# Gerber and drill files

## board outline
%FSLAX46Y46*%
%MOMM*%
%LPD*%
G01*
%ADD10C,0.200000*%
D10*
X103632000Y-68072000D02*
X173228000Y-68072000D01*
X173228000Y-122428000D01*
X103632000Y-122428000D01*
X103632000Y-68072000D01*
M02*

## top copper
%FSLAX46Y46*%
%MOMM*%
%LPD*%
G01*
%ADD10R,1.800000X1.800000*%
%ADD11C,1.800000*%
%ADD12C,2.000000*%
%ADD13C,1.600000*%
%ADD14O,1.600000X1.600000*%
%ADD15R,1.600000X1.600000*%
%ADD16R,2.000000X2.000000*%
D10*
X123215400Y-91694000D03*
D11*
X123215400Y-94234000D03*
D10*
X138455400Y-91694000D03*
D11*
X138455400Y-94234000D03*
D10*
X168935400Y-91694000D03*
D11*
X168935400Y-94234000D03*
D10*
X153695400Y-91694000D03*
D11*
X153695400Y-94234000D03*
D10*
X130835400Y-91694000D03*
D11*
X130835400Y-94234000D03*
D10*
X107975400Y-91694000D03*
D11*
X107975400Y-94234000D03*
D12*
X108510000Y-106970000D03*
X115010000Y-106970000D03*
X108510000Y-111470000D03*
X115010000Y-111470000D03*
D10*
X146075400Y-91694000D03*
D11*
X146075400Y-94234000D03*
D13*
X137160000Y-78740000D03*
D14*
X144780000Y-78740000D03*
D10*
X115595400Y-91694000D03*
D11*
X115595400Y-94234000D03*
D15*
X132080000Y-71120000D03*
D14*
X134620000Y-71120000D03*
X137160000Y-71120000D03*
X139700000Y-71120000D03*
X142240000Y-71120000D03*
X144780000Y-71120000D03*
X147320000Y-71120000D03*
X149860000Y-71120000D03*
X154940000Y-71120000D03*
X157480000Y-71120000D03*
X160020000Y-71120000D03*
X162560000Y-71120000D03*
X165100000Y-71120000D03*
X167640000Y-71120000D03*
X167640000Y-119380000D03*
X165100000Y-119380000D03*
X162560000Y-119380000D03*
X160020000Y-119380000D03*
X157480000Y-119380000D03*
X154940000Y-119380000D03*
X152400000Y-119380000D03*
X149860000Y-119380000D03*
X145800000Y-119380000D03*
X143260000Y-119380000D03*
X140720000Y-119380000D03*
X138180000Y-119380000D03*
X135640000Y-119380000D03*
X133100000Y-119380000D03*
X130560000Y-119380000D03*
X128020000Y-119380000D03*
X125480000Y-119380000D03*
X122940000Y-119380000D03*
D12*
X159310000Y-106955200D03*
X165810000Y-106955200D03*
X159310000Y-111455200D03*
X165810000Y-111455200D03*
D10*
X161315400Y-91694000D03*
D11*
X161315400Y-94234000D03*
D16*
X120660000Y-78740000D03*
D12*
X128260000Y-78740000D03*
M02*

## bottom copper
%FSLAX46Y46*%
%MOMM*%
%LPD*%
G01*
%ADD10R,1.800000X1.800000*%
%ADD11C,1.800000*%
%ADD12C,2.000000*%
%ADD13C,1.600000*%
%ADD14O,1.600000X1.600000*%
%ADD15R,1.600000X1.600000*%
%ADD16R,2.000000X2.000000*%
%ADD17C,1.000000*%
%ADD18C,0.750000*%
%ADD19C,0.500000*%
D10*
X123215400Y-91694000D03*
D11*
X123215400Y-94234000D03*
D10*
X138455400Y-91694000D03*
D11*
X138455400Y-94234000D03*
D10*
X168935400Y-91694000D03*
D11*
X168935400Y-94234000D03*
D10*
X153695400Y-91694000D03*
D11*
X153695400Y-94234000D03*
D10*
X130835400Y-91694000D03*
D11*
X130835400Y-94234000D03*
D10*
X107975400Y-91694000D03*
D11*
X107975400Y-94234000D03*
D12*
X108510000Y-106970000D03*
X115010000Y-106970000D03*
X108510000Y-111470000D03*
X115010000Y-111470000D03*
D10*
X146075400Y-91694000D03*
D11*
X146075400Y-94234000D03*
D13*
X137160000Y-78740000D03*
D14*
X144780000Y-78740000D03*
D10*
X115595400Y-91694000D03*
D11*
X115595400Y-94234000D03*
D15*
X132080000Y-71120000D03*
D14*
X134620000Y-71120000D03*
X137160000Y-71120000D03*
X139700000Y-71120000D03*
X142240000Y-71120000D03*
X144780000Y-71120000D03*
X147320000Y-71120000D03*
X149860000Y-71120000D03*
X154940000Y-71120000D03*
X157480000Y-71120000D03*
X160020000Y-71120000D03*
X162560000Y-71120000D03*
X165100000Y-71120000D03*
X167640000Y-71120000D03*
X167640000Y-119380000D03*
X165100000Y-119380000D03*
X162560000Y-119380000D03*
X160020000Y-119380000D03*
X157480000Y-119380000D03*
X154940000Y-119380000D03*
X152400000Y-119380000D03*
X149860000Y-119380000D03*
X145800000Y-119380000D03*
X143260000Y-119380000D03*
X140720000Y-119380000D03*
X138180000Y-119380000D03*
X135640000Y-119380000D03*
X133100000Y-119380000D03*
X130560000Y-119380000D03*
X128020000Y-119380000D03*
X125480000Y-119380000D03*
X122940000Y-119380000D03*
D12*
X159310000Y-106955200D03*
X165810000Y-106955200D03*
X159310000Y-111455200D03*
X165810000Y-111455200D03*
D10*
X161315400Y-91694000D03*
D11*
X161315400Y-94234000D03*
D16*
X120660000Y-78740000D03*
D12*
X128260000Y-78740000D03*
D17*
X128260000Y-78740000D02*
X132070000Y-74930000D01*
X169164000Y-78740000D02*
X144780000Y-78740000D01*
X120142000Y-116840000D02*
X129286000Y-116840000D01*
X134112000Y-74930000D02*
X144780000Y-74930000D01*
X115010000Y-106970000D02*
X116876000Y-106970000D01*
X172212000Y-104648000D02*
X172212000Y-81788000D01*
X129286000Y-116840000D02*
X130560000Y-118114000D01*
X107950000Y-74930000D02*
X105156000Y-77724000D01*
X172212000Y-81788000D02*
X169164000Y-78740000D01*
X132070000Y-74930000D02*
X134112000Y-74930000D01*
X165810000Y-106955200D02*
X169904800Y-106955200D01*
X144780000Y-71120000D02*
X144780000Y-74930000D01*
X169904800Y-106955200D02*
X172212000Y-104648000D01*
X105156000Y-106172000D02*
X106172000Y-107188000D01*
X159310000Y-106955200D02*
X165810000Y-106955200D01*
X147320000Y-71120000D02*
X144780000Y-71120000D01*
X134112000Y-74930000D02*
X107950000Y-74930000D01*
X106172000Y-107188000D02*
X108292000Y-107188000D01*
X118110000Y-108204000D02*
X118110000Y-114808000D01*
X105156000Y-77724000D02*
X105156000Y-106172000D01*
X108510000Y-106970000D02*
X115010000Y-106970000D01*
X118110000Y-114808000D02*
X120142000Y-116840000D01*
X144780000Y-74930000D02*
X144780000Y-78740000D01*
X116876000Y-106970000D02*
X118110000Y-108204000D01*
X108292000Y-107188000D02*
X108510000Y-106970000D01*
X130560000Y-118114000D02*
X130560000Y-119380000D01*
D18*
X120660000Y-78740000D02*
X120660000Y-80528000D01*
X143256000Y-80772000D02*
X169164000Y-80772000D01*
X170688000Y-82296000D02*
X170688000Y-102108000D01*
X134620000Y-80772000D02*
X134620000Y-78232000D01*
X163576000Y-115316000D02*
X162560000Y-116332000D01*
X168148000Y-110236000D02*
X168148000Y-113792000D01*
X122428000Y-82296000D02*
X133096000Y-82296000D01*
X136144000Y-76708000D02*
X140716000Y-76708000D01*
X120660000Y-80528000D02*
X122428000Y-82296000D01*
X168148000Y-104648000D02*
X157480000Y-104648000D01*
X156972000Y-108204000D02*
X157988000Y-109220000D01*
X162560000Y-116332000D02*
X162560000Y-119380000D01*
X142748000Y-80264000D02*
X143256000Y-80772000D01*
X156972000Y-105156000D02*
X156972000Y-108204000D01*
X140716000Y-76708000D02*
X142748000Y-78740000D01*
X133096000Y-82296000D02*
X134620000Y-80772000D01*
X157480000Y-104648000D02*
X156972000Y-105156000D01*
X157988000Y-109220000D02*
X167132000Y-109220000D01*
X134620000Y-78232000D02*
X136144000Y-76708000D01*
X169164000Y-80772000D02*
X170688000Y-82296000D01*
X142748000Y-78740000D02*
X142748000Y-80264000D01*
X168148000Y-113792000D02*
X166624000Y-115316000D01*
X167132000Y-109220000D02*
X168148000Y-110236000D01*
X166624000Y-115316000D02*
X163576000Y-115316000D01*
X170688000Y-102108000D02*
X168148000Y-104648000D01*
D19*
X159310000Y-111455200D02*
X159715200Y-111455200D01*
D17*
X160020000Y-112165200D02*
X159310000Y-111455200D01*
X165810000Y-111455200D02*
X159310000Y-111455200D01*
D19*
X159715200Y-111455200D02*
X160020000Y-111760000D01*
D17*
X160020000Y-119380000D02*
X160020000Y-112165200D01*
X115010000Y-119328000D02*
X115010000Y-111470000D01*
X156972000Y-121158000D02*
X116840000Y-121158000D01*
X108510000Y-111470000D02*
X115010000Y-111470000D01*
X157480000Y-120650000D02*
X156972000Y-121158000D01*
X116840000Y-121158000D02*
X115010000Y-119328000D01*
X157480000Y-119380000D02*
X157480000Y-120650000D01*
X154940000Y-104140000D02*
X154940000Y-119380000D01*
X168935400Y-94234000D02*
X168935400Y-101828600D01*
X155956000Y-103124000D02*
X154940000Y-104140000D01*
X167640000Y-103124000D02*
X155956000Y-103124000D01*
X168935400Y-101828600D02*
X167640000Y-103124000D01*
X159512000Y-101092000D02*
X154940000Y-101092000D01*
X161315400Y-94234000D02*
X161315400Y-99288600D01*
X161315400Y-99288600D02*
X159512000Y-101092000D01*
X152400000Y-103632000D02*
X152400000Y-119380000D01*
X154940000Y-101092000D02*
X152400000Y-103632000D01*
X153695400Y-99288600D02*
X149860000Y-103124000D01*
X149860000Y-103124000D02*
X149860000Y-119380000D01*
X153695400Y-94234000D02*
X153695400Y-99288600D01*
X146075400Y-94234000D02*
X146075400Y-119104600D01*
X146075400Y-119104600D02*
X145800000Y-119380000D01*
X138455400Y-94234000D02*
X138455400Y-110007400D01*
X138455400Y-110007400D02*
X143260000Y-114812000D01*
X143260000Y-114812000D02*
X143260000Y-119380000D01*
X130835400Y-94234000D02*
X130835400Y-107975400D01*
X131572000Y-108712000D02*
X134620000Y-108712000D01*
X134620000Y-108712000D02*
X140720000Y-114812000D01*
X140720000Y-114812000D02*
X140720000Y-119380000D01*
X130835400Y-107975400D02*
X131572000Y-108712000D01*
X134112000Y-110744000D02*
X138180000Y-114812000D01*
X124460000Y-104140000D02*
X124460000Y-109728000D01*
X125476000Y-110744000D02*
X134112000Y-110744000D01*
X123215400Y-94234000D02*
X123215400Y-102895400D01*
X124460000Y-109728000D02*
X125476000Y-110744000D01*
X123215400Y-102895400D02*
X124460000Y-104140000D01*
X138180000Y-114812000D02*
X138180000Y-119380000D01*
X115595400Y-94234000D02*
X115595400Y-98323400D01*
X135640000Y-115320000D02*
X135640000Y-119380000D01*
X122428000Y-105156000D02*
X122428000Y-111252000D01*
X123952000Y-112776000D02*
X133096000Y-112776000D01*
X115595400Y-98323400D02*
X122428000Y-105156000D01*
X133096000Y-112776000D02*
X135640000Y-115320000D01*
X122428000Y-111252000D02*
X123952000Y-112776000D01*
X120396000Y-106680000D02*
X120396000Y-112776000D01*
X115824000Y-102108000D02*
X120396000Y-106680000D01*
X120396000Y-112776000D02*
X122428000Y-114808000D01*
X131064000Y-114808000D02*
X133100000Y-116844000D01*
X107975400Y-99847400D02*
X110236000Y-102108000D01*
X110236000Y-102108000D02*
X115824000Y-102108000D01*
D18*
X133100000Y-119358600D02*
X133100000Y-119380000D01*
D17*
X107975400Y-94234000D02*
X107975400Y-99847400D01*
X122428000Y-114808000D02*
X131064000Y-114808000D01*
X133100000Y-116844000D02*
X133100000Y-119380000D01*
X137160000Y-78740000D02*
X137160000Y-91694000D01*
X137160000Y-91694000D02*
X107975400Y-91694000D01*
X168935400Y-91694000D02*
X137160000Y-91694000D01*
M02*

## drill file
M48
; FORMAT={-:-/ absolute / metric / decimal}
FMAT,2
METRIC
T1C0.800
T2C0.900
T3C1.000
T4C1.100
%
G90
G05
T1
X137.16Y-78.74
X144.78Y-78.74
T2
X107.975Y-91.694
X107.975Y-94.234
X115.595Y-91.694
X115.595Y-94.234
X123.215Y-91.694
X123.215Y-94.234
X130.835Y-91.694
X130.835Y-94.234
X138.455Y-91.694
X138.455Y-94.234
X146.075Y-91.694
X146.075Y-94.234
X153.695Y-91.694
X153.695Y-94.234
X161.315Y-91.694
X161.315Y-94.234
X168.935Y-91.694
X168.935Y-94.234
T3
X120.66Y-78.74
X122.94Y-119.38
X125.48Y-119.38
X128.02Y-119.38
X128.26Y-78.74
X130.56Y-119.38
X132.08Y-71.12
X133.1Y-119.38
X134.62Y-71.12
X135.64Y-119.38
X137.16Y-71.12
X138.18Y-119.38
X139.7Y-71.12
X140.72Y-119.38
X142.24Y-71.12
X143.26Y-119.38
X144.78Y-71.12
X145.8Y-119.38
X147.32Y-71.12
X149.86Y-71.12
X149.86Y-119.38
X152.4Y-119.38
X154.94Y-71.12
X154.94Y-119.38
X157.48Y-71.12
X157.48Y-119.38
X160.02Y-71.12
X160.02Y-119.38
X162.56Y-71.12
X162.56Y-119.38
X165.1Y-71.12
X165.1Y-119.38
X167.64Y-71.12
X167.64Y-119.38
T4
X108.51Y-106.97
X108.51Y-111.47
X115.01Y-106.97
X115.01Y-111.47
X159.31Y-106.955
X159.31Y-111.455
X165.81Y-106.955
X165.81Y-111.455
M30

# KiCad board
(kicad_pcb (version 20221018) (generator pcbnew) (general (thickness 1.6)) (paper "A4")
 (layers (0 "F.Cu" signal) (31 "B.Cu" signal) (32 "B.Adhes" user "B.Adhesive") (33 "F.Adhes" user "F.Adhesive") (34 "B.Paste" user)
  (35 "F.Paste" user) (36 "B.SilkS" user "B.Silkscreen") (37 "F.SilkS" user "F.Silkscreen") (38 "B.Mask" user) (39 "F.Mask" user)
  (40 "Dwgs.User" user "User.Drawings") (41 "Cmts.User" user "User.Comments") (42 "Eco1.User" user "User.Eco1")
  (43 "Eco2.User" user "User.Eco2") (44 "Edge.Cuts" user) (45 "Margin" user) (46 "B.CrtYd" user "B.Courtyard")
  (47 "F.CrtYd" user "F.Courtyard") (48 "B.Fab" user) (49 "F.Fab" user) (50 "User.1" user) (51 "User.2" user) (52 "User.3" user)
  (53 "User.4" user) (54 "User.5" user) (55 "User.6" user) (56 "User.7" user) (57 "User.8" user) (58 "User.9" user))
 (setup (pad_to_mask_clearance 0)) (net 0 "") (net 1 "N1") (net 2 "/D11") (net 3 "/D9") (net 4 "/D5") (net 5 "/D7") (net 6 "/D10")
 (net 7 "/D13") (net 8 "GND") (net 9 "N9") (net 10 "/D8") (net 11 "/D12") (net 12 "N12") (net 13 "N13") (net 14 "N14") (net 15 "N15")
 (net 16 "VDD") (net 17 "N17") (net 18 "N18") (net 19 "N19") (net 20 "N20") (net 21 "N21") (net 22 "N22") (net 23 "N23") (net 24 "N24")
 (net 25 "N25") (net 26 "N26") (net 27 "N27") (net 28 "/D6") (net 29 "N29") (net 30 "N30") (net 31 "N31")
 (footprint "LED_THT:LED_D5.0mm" (layer "F.Cu") (at 123.2154 91.694 -90)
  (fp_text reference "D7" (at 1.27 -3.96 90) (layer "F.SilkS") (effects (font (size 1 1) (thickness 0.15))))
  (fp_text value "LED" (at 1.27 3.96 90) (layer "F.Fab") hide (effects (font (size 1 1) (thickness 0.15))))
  (pad "1" thru_hole rect (at 0 0 270) (size 1.8 1.8) (drill 0.9) (layers "*.Cu" "*.Mask") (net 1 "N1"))
  (pad "2" thru_hole circle (at 2.54 0 270) (size 1.8 1.8) (drill 0.9) (layers "*.Cu" "*.Mask") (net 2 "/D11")))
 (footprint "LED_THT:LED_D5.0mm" (layer "F.Cu") (at 138.4554 91.694 -90)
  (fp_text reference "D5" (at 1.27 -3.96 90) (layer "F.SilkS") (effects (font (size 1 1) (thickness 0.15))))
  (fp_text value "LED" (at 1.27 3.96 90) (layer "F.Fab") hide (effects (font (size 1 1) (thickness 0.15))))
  (pad "1" thru_hole rect (at 0 0 270) (size 1.8 1.8) (drill 0.9) (layers "*.Cu" "*.Mask") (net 1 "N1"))
  (pad "2" thru_hole circle (at 2.54 0 270) (size 1.8 1.8) (drill 0.9) (layers "*.Cu" "*.Mask") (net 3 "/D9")))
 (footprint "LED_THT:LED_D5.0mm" (layer "F.Cu") (at 168.9354 91.694 -90)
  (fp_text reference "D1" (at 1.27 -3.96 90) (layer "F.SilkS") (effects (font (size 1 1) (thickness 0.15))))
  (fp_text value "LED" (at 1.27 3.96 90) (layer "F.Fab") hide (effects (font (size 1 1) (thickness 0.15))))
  (pad "1" thru_hole rect (at 0 0 270) (size 1.8 1.8) (drill 0.9) (layers "*.Cu" "*.Mask") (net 1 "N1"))
  (pad "2" thru_hole circle (at 2.54 0 270) (size 1.8 1.8) (drill 0.9) (layers "*.Cu" "*.Mask") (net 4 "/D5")))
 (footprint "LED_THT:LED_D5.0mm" (layer "F.Cu") (at 153.6954 91.694 -90)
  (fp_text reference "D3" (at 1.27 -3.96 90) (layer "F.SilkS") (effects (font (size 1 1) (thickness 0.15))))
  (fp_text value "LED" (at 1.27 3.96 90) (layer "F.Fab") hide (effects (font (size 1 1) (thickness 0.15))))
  (pad "1" thru_hole rect (at 0 0 270) (size 1.8 1.8) (drill 0.9) (layers "*.Cu" "*.Mask") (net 1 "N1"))
  (pad "2" thru_hole circle (at 2.54 0 270) (size 1.8 1.8) (drill 0.9) (layers "*.Cu" "*.Mask") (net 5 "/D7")))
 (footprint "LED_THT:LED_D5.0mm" (layer "F.Cu") (at 130.8354 91.694 -90)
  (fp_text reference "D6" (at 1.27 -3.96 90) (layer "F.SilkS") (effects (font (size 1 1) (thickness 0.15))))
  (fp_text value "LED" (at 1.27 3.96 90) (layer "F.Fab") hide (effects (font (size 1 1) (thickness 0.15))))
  (pad "1" thru_hole rect (at 0 0 270) (size 1.8 1.8) (drill 0.9) (layers "*.Cu" "*.Mask") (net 1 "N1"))
  (pad "2" thru_hole circle (at 2.54 0 270) (size 1.8 1.8) (drill 0.9) (layers "*.Cu" "*.Mask") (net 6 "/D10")))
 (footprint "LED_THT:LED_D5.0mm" (layer "F.Cu") (at 107.9754 91.694 -90)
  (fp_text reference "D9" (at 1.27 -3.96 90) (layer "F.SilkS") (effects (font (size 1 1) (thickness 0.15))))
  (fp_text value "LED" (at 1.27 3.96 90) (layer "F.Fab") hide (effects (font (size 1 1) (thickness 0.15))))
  (pad "1" thru_hole rect (at 0 0 270) (size 1.8 1.8) (drill 0.9) (layers "*.Cu" "*.Mask") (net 1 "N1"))
  (pad "2" thru_hole circle (at 2.54 0 270) (size 1.8 1.8) (drill 0.9) (layers "*.Cu" "*.Mask") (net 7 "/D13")))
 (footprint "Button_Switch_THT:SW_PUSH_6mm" (layer "F.Cu") (at 108.51 106.97)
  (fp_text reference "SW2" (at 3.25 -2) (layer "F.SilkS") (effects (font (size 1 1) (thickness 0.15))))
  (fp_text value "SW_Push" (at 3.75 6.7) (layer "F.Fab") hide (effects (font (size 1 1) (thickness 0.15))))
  (pad "1" thru_hole circle (at 0 0 90) (size 2 2) (drill 1.1) (layers "*.Cu" "*.Mask") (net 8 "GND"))
  (pad "1" thru_hole circle (at 6.5 0 90) (size 2 2) (drill 1.1) (layers "*.Cu" "*.Mask") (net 8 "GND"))
  (pad "2" thru_hole circle (at 0 4.5 90) (size 2 2) (drill 1.1) (layers "*.Cu" "*.Mask") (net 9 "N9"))
  (pad "2" thru_hole circle (at 6.5 4.5 90) (size 2 2) (drill 1.1) (layers "*.Cu" "*.Mask") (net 9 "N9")))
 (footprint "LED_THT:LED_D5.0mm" (layer "F.Cu") (at 146.0754 91.694 -90)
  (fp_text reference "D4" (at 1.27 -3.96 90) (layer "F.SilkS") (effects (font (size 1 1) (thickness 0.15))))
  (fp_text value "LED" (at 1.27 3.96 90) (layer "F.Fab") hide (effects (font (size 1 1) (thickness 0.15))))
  (pad "1" thru_hole rect (at 0 0 270) (size 1.8 1.8) (drill 0.9) (layers "*.Cu" "*.Mask") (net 1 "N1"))
  (pad "2" thru_hole circle (at 2.54 0 270) (size 1.8 1.8) (drill 0.9) (layers "*.Cu" "*.Mask") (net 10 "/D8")))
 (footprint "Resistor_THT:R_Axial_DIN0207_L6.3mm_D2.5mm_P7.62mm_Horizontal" (layer "F.Cu") (at 137.16 78.74)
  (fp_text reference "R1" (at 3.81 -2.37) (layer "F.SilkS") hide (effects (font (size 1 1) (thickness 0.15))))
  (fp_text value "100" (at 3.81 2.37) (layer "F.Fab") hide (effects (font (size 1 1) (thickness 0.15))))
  (pad "1" thru_hole circle (at 0 0) (size 1.6 1.6) (drill 0.8) (layers "*.Cu" "*.Mask") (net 1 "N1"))
  (pad "2" thru_hole oval (at 7.62 0) (size 1.6 1.6) (drill 0.8) (layers "*.Cu" "*.Mask") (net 8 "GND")))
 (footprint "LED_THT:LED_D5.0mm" (layer "F.Cu") (at 115.5954 91.694 -90)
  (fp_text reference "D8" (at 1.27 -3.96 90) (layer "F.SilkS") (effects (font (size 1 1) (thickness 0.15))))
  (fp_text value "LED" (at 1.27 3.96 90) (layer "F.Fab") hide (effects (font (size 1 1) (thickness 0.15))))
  (pad "1" thru_hole rect (at 0 0 270) (size 1.8 1.8) (drill 0.9) (layers "*.Cu" "*.Mask") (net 1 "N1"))
  (pad "2" thru_hole circle (at 2.54 0 270) (size 1.8 1.8) (drill 0.9) (layers "*.Cu" "*.Mask") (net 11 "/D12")))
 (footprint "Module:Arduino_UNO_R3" (layer "F.Cu") (at 132.08 71.12)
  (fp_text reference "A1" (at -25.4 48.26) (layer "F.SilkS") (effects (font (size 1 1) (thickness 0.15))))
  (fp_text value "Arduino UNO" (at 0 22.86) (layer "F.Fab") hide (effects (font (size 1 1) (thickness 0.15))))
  (pad "1" thru_hole rect (at 0 0 90) (size 1.6 1.6) (drill 1) (layers "*.Cu" "*.Mask") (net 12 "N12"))
  (pad "2" thru_hole oval (at 2.54 0 90) (size 1.6 1.6) (drill 1) (layers "*.Cu" "*.Mask") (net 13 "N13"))
  (pad "3" thru_hole oval (at 5.08 0 90) (size 1.6 1.6) (drill 1) (layers "*.Cu" "*.Mask") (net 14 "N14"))
  (pad "4" thru_hole oval (at 7.62 0 90) (size 1.6 1.6) (drill 1) (layers "*.Cu" "*.Mask") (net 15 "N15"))
  (pad "5" thru_hole oval (at 10.16 0 90) (size 1.6 1.6) (drill 1) (layers "*.Cu" "*.Mask") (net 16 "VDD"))
  (pad "6" thru_hole oval (at 12.7 0 90) (size 1.6 1.6) (drill 1) (layers "*.Cu" "*.Mask") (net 8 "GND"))
  (pad "7" thru_hole oval (at 15.24 0 90) (size 1.6 1.6) (drill 1) (layers "*.Cu" "*.Mask") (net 8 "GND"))
  (pad "8" thru_hole oval (at 17.78 0 90) (size 1.6 1.6) (drill 1) (layers "*.Cu" "*.Mask") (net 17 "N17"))
  (pad "9" thru_hole oval (at 22.86 0 90) (size 1.6 1.6) (drill 1) (layers "*.Cu" "*.Mask") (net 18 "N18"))
  (pad "10" thru_hole oval (at 25.4 0 90) (size 1.6 1.6) (drill 1) (layers "*.Cu" "*.Mask") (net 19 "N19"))
  (pad "11" thru_hole oval (at 27.94 0 90) (size 1.6 1.6) (drill 1) (layers "*.Cu" "*.Mask") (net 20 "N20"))
  (pad "12" thru_hole oval (at 30.48 0 90) (size 1.6 1.6) (drill 1) (layers "*.Cu" "*.Mask") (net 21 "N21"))
  (pad "13" thru_hole oval (at 33.02 0 90) (size 1.6 1.6) (drill 1) (layers "*.Cu" "*.Mask") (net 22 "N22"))
  (pad "14" thru_hole oval (at 35.56 0 90) (size 1.6 1.6) (drill 1) (layers "*.Cu" "*.Mask") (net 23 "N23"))
  (pad "15" thru_hole oval (at 35.56 48.26 90) (size 1.6 1.6) (drill 1) (layers "*.Cu" "*.Mask") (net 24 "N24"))
  (pad "16" thru_hole oval (at 33.02 48.26 90) (size 1.6 1.6) (drill 1) (layers "*.Cu" "*.Mask") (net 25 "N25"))
  (pad "17" thru_hole oval (at 30.48 48.26 90) (size 1.6 1.6) (drill 1) (layers "*.Cu" "*.Mask") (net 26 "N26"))
  (pad "18" thru_hole oval (at 27.94 48.26 90) (size 1.6 1.6) (drill 1) (layers "*.Cu" "*.Mask") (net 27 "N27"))
  (pad "19" thru_hole oval (at 25.4 48.26 90) (size 1.6 1.6) (drill 1) (layers "*.Cu" "*.Mask") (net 9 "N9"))
  (pad "20" thru_hole oval (at 22.86 48.26 90) (size 1.6 1.6) (drill 1) (layers "*.Cu" "*.Mask") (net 4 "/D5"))
  (pad "21" thru_hole oval (at 20.32 48.26 90) (size 1.6 1.6) (drill 1) (layers "*.Cu" "*.Mask") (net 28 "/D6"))
  (pad "22" thru_hole oval (at 17.78 48.26 90) (size 1.6 1.6) (drill 1) (layers "*.Cu" "*.Mask") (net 5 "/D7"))
  (pad "23" thru_hole oval (at 13.72 48.26 90) (size 1.6 1.6) (drill 1) (layers "*.Cu" "*.Mask") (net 10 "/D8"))
  (pad "24" thru_hole oval (at 11.18 48.26 90) (size 1.6 1.6) (drill 1) (layers "*.Cu" "*.Mask") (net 3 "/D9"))
  (pad "25" thru_hole oval (at 8.64 48.26 90) (size 1.6 1.6) (drill 1) (layers "*.Cu" "*.Mask") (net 6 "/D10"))
  (pad "26" thru_hole oval (at 6.1 48.26 90) (size 1.6 1.6) (drill 1) (layers "*.Cu" "*.Mask") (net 2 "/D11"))
  (pad "27" thru_hole oval (at 3.56 48.26 90) (size 1.6 1.6) (drill 1) (layers "*.Cu" "*.Mask") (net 11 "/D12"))
  (pad "28" thru_hole oval (at 1.02 48.26 90) (size 1.6 1.6) (drill 1) (layers "*.Cu" "*.Mask") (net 7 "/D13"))
  (pad "29" thru_hole oval (at -1.52 48.26 90) (size 1.6 1.6) (drill 1) (layers "*.Cu" "*.Mask") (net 8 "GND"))
  (pad "30" thru_hole oval (at -4.06 48.26 90) (size 1.6 1.6) (drill 1) (layers "*.Cu" "*.Mask") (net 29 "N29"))
  (pad "31" thru_hole oval (at -6.6 48.26 90) (size 1.6 1.6) (drill 1) (layers "*.Cu" "*.Mask") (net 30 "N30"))
  (pad "32" thru_hole oval (at -9.14 48.26 90) (size 1.6 1.6) (drill 1) (layers "*.Cu" "*.Mask") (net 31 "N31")))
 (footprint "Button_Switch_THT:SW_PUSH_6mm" (layer "F.Cu") (at 159.31 106.9552)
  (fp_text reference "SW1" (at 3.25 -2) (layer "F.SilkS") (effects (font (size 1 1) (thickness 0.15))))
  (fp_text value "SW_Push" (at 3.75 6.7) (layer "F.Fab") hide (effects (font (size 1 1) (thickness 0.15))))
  (pad "1" thru_hole circle (at 0 0 90) (size 2 2) (drill 1.1) (layers "*.Cu" "*.Mask") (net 8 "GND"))
  (pad "1" thru_hole circle (at 6.5 0 90) (size 2 2) (drill 1.1) (layers "*.Cu" "*.Mask") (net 8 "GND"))
  (pad "2" thru_hole circle (at 0 4.5 90) (size 2 2) (drill 1.1) (layers "*.Cu" "*.Mask") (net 27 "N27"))
  (pad "2" thru_hole circle (at 6.5 4.5 90) (size 2 2) (drill 1.1) (layers "*.Cu" "*.Mask") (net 27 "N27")))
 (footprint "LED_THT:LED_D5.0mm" (layer "F.Cu") (at 161.3154 91.694 -90)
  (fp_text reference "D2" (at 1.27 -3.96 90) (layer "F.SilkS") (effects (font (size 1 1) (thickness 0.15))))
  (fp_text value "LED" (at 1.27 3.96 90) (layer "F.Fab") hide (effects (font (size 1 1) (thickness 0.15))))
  (pad "1" thru_hole rect (at 0 0 270) (size 1.8 1.8) (drill 0.9) (layers "*.Cu" "*.Mask") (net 1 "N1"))
  (pad "2" thru_hole circle (at 2.54 0 270) (size 1.8 1.8) (drill 0.9) (layers "*.Cu" "*.Mask") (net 28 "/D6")))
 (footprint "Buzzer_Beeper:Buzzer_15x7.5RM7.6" (layer "F.Cu") (at 120.66 78.74)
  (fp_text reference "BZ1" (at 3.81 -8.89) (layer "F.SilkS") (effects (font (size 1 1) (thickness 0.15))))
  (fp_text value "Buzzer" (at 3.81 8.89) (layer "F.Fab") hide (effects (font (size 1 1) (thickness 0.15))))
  (pad "1" thru_hole rect (at 0 0) (size 2 2) (drill 1) (layers "*.Cu" "*.Mask") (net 26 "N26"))
  (pad "2" thru_hole circle (at 7.6 0) (size 2 2) (drill 1) (layers "*.Cu" "*.Mask") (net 8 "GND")))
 (gr_rect (start 103.632 68.072) (end 173.228 122.428) (stroke (width 0.2) (type default)) (fill none) (layer "Edge.Cuts"))
 (segment (start 128.26 78.74) (end 132.07 74.93) (width 1) (layer "B.Cu") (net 8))
 (segment (start 169.164 78.74) (end 144.78 78.74) (width 1) (layer "B.Cu") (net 8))
 (segment (start 120.142 116.84) (end 129.286 116.84) (width 1) (layer "B.Cu") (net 8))
 (segment (start 134.112 74.93) (end 144.78 74.93) (width 1) (layer "B.Cu") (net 8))
 (segment (start 115.01 106.97) (end 116.876 106.97) (width 1) (layer "B.Cu") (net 8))
 (segment (start 172.212 104.648) (end 172.212 81.788) (width 1) (layer "B.Cu") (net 8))
 (segment (start 129.286 116.84) (end 130.56 118.114) (width 1) (layer "B.Cu") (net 8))
 (segment (start 107.95 74.93) (end 105.156 77.724) (width 1) (layer "B.Cu") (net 8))
 (segment (start 172.212 81.788) (end 169.164 78.74) (width 1) (layer "B.Cu") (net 8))
 (segment (start 132.07 74.93) (end 134.112 74.93) (width 1) (layer "B.Cu") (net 8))
 (segment (start 165.81 106.9552) (end 169.9048 106.9552) (width 1) (layer "B.Cu") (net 8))
 (segment (start 144.78 71.12) (end 144.78 74.93) (width 1) (layer "B.Cu") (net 8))
 (segment (start 169.9048 106.9552) (end 172.212 104.648) (width 1) (layer "B.Cu") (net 8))
 (segment (start 105.156 106.172) (end 106.172 107.188) (width 1) (layer "B.Cu") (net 8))
 (segment (start 159.31 106.9552) (end 165.81 106.9552) (width 1) (layer "B.Cu") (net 8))
 (segment (start 147.32 71.12) (end 144.78 71.12) (width 1) (layer "B.Cu") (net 8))
 (segment (start 134.112 74.93) (end 107.95 74.93) (width 1) (layer "B.Cu") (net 8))
 (segment (start 106.172 107.188) (end 108.292 107.188) (width 1) (layer "B.Cu") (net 8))
 (segment (start 118.11 108.204) (end 118.11 114.808) (width 1) (layer "B.Cu") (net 8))
 (segment (start 105.156 77.724) (end 105.156 106.172) (width 1) (layer "B.Cu") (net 8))
 (segment (start 108.51 106.97) (end 115.01 106.97) (width 1) (layer "B.Cu") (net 8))
 (segment (start 118.11 114.808) (end 120.142 116.84) (width 1) (layer "B.Cu") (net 8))
 (segment (start 144.78 74.93) (end 144.78 78.74) (width 1) (layer "B.Cu") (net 8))
 (segment (start 116.876 106.97) (end 118.11 108.204) (width 1) (layer "B.Cu") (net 8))
 (segment (start 108.292 107.188) (end 108.51 106.97) (width 1) (layer "B.Cu") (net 8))
 (segment (start 130.56 118.114) (end 130.56 119.38) (width 1) (layer "B.Cu") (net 8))
 (segment (start 120.66 78.74) (end 120.66 80.528) (width 0.75) (layer "B.Cu") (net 26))
 (segment (start 143.256 80.772) (end 169.164 80.772) (width 0.75) (layer "B.Cu") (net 26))
 (segment (start 170.688 82.296) (end 170.688 102.108) (width 0.75) (layer "B.Cu") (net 26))
 (segment (start 134.62 80.772) (end 134.62 78.232) (width 0.75) (layer "B.Cu") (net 26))
 (segment (start 163.576 115.316) (end 162.56 116.332) (width 0.75) (layer "B.Cu") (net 26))
 (segment (start 168.148 110.236) (end 168.148 113.792) (width 0.75) (layer "B.Cu") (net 26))
 (segment (start 122.428 82.296) (end 133.096 82.296) (width 0.75) (layer "B.Cu") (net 26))
 (segment (start 136.144 76.708) (end 140.716 76.708) (width 0.75) (layer "B.Cu") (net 26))
 (segment (start 120.66 80.528) (end 122.428 82.296) (width 0.75) (layer "B.Cu") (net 26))
 (segment (start 168.148 104.648) (end 157.48 104.648) (width 0.75) (layer "B.Cu") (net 26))
 (segment (start 156.972 108.204) (end 157.988 109.22) (width 0.75) (layer "B.Cu") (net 26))
 (segment (start 162.56 116.332) (end 162.56 119.38) (width 0.75) (layer "B.Cu") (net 26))
 (segment (start 142.748 80.264) (end 143.256 80.772) (width 0.75) (layer "B.Cu") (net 26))
 (segment (start 156.972 105.156) (end 156.972 108.204) (width 0.75) (layer "B.Cu") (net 26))
 (segment (start 140.716 76.708) (end 142.748 78.74) (width 0.75) (layer "B.Cu") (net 26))
 (segment (start 133.096 82.296) (end 134.62 80.772) (width 0.75) (layer "B.Cu") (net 26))
 (segment (start 157.48 104.648) (end 156.972 105.156) (width 0.75) (layer "B.Cu") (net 26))
 (segment (start 157.988 109.22) (end 167.132 109.22) (width 0.75) (layer "B.Cu") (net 26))
 (segment (start 134.62 78.232) (end 136.144 76.708) (width 0.75) (layer "B.Cu") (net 26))
 (segment (start 169.164 80.772) (end 170.688 82.296) (width 0.75) (layer "B.Cu") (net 26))
 (segment (start 142.748 78.74) (end 142.748 80.264) (width 0.75) (layer "B.Cu") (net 26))
 (segment (start 168.148 113.792) (end 166.624 115.316) (width 0.75) (layer "B.Cu") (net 26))
 (segment (start 167.132 109.22) (end 168.148 110.236) (width 0.75) (layer "B.Cu") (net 26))
 (segment (start 166.624 115.316) (end 163.576 115.316) (width 0.75) (layer "B.Cu") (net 26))
 (segment (start 170.688 102.108) (end 168.148 104.648) (width 0.75) (layer "B.Cu") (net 26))
 (segment (start 159.31 111.4552) (end 159.7152 111.4552) (width 0.5) (layer "B.Cu") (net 27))
 (segment (start 160.02 112.1652) (end 159.31 111.4552) (width 1) (layer "B.Cu") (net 27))
 (segment (start 165.81 111.4552) (end 159.31 111.4552) (width 1) (layer "B.Cu") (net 27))
 (segment (start 159.7152 111.4552) (end 160.02 111.76) (width 0.5) (layer "B.Cu") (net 27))
 (segment (start 160.02 119.38) (end 160.02 112.1652) (width 1) (layer "B.Cu") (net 27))
 (segment (start 115.01 119.328) (end 115.01 111.47) (width 1) (layer "B.Cu") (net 9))
 (segment (start 156.972 121.158) (end 116.84 121.158) (width 1) (layer "B.Cu") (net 9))
 (segment (start 108.51 111.47) (end 115.01 111.47) (width 1) (layer "B.Cu") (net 9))
 (segment (start 157.48 120.65) (end 156.972 121.158) (width 1) (layer "B.Cu") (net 9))
 (segment (start 116.84 121.158) (end 115.01 119.328) (width 1) (layer "B.Cu") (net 9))
 (segment (start 157.48 119.38) (end 157.48 120.65) (width 1) (layer "B.Cu") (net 9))
 (segment (start 154.94 104.14) (end 154.94 119.38) (width 1) (layer "B.Cu") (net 4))
 (segment (start 168.9354 94.234) (end 168.9354 101.8286) (width 1) (layer "B.Cu") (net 4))
 (segment (start 155.956 103.124) (end 154.94 104.14) (width 1) (layer "B.Cu") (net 4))
 (segment (start 167.64 103.124) (end 155.956 103.124) (width 1) (layer "B.Cu") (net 4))
 (segment (start 168.9354 101.8286) (end 167.64 103.124) (width 1) (layer "B.Cu") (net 4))
 (segment (start 159.512 101.092) (end 154.94 101.092) (width 1) (layer "B.Cu") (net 28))
 (segment (start 161.3154 94.234) (end 161.3154 99.2886) (width 1) (layer "B.Cu") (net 28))
 (segment (start 161.3154 99.2886) (end 159.512 101.092) (width 1) (layer "B.Cu") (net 28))
 (segment (start 152.4 103.632) (end 152.4 119.38) (width 1) (layer "B.Cu") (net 28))
 (segment (start 154.94 101.092) (end 152.4 103.632) (width 1) (layer "B.Cu") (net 28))
 (segment (start 153.6954 99.2886) (end 149.86 103.124) (width 1) (layer "B.Cu") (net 5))
 (segment (start 149.86 103.124) (end 149.86 119.38) (width 1) (layer "B.Cu") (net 5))
 (segment (start 153.6954 94.234) (end 153.6954 99.2886) (width 1) (layer "B.Cu") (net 5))
 (segment (start 146.0754 94.234) (end 146.0754 119.1046) (width 1) (layer "B.Cu") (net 10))
 (segment (start 146.0754 119.1046) (end 145.8 119.38) (width 1) (layer "B.Cu") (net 10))
 (segment (start 138.4554 94.234) (end 138.4554 110.0074) (width 1) (layer "B.Cu") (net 3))
 (segment (start 138.4554 110.0074) (end 143.26 114.812) (width 1) (layer "B.Cu") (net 3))
 (segment (start 143.26 114.812) (end 143.26 119.38) (width 1) (layer "B.Cu") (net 3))
 (segment (start 130.8354 94.234) (end 130.8354 107.9754) (width 1) (layer "B.Cu") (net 6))
 (segment (start 131.572 108.712) (end 134.62 108.712) (width 1) (layer "B.Cu") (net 6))
 (segment (start 134.62 108.712) (end 140.72 114.812) (width 1) (layer "B.Cu") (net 6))
 (segment (start 140.72 114.812) (end 140.72 119.38) (width 1) (layer "B.Cu") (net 6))
 (segment (start 130.8354 107.9754) (end 131.572 108.712) (width 1) (layer "B.Cu") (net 6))
 (segment (start 134.112 110.744) (end 138.18 114.812) (width 1) (layer "B.Cu") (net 2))
 (segment (start 124.46 104.14) (end 124.46 109.728) (width 1) (layer "B.Cu") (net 2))
 (segment (start 125.476 110.744) (end 134.112 110.744) (width 1) (layer "B.Cu") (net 2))
 (segment (start 123.2154 94.234) (end 123.2154 102.8954) (width 1) (layer "B.Cu") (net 2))
 (segment (start 124.46 109.728) (end 125.476 110.744) (width 1) (layer "B.Cu") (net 2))
 (segment (start 123.2154 102.8954) (end 124.46 104.14) (width 1) (layer "B.Cu") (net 2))
 (segment (start 138.18 114.812) (end 138.18 119.38) (width 1) (layer "B.Cu") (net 2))
 (segment (start 115.5954 94.234) (end 115.5954 98.3234) (width 1) (layer "B.Cu") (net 11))
 (segment (start 135.64 115.32) (end 135.64 119.38) (width 1) (layer "B.Cu") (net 11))
 (segment (start 122.428 105.156) (end 122.428 111.252) (width 1) (layer "B.Cu") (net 11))
 (segment (start 123.952 112.776) (end 133.096 112.776) (width 1) (layer "B.Cu") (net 11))
 (segment (start 115.5954 98.3234) (end 122.428 105.156) (width 1) (layer "B.Cu") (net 11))
 (segment (start 133.096 112.776) (end 135.64 115.32) (width 1) (layer "B.Cu") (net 11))
 (segment (start 122.428 111.252) (end 123.952 112.776) (width 1) (layer "B.Cu") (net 11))
 (segment (start 120.396 106.68) (end 120.396 112.776) (width 1) (layer "B.Cu") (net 7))
 (segment (start 115.824 102.108) (end 120.396 106.68) (width 1) (layer "B.Cu") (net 7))
 (segment (start 120.396 112.776) (end 122.428 114.808) (width 1) (layer "B.Cu") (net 7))
 (segment (start 131.064 114.808) (end 133.1 116.844) (width 1) (layer "B.Cu") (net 7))
 (segment (start 107.9754 99.8474) (end 110.236 102.108) (width 1) (layer "B.Cu") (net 7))
 (segment (start 110.236 102.108) (end 115.824 102.108) (width 1) (layer "B.Cu") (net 7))
 (segment (start 133.1 119.3586) (end 133.1 119.38) (width 0.75) (layer "B.Cu") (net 7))
 (segment (start 107.9754 94.234) (end 107.9754 99.8474) (width 1) (layer "B.Cu") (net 7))
 (segment (start 122.428 114.808) (end 131.064 114.808) (width 1) (layer "B.Cu") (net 7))
 (segment (start 133.1 116.844) (end 133.1 119.38) (width 1) (layer "B.Cu") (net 7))
 (segment (start 137.16 78.74) (end 137.16 91.694) (width 1) (layer "B.Cu") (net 1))
 (segment (start 137.16 91.694) (end 107.9754 91.694) (width 1) (layer "B.Cu") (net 1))
 (segment (start 168.9354 91.694) (end 137.16 91.694) (width 1) (layer "B.Cu") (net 1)))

